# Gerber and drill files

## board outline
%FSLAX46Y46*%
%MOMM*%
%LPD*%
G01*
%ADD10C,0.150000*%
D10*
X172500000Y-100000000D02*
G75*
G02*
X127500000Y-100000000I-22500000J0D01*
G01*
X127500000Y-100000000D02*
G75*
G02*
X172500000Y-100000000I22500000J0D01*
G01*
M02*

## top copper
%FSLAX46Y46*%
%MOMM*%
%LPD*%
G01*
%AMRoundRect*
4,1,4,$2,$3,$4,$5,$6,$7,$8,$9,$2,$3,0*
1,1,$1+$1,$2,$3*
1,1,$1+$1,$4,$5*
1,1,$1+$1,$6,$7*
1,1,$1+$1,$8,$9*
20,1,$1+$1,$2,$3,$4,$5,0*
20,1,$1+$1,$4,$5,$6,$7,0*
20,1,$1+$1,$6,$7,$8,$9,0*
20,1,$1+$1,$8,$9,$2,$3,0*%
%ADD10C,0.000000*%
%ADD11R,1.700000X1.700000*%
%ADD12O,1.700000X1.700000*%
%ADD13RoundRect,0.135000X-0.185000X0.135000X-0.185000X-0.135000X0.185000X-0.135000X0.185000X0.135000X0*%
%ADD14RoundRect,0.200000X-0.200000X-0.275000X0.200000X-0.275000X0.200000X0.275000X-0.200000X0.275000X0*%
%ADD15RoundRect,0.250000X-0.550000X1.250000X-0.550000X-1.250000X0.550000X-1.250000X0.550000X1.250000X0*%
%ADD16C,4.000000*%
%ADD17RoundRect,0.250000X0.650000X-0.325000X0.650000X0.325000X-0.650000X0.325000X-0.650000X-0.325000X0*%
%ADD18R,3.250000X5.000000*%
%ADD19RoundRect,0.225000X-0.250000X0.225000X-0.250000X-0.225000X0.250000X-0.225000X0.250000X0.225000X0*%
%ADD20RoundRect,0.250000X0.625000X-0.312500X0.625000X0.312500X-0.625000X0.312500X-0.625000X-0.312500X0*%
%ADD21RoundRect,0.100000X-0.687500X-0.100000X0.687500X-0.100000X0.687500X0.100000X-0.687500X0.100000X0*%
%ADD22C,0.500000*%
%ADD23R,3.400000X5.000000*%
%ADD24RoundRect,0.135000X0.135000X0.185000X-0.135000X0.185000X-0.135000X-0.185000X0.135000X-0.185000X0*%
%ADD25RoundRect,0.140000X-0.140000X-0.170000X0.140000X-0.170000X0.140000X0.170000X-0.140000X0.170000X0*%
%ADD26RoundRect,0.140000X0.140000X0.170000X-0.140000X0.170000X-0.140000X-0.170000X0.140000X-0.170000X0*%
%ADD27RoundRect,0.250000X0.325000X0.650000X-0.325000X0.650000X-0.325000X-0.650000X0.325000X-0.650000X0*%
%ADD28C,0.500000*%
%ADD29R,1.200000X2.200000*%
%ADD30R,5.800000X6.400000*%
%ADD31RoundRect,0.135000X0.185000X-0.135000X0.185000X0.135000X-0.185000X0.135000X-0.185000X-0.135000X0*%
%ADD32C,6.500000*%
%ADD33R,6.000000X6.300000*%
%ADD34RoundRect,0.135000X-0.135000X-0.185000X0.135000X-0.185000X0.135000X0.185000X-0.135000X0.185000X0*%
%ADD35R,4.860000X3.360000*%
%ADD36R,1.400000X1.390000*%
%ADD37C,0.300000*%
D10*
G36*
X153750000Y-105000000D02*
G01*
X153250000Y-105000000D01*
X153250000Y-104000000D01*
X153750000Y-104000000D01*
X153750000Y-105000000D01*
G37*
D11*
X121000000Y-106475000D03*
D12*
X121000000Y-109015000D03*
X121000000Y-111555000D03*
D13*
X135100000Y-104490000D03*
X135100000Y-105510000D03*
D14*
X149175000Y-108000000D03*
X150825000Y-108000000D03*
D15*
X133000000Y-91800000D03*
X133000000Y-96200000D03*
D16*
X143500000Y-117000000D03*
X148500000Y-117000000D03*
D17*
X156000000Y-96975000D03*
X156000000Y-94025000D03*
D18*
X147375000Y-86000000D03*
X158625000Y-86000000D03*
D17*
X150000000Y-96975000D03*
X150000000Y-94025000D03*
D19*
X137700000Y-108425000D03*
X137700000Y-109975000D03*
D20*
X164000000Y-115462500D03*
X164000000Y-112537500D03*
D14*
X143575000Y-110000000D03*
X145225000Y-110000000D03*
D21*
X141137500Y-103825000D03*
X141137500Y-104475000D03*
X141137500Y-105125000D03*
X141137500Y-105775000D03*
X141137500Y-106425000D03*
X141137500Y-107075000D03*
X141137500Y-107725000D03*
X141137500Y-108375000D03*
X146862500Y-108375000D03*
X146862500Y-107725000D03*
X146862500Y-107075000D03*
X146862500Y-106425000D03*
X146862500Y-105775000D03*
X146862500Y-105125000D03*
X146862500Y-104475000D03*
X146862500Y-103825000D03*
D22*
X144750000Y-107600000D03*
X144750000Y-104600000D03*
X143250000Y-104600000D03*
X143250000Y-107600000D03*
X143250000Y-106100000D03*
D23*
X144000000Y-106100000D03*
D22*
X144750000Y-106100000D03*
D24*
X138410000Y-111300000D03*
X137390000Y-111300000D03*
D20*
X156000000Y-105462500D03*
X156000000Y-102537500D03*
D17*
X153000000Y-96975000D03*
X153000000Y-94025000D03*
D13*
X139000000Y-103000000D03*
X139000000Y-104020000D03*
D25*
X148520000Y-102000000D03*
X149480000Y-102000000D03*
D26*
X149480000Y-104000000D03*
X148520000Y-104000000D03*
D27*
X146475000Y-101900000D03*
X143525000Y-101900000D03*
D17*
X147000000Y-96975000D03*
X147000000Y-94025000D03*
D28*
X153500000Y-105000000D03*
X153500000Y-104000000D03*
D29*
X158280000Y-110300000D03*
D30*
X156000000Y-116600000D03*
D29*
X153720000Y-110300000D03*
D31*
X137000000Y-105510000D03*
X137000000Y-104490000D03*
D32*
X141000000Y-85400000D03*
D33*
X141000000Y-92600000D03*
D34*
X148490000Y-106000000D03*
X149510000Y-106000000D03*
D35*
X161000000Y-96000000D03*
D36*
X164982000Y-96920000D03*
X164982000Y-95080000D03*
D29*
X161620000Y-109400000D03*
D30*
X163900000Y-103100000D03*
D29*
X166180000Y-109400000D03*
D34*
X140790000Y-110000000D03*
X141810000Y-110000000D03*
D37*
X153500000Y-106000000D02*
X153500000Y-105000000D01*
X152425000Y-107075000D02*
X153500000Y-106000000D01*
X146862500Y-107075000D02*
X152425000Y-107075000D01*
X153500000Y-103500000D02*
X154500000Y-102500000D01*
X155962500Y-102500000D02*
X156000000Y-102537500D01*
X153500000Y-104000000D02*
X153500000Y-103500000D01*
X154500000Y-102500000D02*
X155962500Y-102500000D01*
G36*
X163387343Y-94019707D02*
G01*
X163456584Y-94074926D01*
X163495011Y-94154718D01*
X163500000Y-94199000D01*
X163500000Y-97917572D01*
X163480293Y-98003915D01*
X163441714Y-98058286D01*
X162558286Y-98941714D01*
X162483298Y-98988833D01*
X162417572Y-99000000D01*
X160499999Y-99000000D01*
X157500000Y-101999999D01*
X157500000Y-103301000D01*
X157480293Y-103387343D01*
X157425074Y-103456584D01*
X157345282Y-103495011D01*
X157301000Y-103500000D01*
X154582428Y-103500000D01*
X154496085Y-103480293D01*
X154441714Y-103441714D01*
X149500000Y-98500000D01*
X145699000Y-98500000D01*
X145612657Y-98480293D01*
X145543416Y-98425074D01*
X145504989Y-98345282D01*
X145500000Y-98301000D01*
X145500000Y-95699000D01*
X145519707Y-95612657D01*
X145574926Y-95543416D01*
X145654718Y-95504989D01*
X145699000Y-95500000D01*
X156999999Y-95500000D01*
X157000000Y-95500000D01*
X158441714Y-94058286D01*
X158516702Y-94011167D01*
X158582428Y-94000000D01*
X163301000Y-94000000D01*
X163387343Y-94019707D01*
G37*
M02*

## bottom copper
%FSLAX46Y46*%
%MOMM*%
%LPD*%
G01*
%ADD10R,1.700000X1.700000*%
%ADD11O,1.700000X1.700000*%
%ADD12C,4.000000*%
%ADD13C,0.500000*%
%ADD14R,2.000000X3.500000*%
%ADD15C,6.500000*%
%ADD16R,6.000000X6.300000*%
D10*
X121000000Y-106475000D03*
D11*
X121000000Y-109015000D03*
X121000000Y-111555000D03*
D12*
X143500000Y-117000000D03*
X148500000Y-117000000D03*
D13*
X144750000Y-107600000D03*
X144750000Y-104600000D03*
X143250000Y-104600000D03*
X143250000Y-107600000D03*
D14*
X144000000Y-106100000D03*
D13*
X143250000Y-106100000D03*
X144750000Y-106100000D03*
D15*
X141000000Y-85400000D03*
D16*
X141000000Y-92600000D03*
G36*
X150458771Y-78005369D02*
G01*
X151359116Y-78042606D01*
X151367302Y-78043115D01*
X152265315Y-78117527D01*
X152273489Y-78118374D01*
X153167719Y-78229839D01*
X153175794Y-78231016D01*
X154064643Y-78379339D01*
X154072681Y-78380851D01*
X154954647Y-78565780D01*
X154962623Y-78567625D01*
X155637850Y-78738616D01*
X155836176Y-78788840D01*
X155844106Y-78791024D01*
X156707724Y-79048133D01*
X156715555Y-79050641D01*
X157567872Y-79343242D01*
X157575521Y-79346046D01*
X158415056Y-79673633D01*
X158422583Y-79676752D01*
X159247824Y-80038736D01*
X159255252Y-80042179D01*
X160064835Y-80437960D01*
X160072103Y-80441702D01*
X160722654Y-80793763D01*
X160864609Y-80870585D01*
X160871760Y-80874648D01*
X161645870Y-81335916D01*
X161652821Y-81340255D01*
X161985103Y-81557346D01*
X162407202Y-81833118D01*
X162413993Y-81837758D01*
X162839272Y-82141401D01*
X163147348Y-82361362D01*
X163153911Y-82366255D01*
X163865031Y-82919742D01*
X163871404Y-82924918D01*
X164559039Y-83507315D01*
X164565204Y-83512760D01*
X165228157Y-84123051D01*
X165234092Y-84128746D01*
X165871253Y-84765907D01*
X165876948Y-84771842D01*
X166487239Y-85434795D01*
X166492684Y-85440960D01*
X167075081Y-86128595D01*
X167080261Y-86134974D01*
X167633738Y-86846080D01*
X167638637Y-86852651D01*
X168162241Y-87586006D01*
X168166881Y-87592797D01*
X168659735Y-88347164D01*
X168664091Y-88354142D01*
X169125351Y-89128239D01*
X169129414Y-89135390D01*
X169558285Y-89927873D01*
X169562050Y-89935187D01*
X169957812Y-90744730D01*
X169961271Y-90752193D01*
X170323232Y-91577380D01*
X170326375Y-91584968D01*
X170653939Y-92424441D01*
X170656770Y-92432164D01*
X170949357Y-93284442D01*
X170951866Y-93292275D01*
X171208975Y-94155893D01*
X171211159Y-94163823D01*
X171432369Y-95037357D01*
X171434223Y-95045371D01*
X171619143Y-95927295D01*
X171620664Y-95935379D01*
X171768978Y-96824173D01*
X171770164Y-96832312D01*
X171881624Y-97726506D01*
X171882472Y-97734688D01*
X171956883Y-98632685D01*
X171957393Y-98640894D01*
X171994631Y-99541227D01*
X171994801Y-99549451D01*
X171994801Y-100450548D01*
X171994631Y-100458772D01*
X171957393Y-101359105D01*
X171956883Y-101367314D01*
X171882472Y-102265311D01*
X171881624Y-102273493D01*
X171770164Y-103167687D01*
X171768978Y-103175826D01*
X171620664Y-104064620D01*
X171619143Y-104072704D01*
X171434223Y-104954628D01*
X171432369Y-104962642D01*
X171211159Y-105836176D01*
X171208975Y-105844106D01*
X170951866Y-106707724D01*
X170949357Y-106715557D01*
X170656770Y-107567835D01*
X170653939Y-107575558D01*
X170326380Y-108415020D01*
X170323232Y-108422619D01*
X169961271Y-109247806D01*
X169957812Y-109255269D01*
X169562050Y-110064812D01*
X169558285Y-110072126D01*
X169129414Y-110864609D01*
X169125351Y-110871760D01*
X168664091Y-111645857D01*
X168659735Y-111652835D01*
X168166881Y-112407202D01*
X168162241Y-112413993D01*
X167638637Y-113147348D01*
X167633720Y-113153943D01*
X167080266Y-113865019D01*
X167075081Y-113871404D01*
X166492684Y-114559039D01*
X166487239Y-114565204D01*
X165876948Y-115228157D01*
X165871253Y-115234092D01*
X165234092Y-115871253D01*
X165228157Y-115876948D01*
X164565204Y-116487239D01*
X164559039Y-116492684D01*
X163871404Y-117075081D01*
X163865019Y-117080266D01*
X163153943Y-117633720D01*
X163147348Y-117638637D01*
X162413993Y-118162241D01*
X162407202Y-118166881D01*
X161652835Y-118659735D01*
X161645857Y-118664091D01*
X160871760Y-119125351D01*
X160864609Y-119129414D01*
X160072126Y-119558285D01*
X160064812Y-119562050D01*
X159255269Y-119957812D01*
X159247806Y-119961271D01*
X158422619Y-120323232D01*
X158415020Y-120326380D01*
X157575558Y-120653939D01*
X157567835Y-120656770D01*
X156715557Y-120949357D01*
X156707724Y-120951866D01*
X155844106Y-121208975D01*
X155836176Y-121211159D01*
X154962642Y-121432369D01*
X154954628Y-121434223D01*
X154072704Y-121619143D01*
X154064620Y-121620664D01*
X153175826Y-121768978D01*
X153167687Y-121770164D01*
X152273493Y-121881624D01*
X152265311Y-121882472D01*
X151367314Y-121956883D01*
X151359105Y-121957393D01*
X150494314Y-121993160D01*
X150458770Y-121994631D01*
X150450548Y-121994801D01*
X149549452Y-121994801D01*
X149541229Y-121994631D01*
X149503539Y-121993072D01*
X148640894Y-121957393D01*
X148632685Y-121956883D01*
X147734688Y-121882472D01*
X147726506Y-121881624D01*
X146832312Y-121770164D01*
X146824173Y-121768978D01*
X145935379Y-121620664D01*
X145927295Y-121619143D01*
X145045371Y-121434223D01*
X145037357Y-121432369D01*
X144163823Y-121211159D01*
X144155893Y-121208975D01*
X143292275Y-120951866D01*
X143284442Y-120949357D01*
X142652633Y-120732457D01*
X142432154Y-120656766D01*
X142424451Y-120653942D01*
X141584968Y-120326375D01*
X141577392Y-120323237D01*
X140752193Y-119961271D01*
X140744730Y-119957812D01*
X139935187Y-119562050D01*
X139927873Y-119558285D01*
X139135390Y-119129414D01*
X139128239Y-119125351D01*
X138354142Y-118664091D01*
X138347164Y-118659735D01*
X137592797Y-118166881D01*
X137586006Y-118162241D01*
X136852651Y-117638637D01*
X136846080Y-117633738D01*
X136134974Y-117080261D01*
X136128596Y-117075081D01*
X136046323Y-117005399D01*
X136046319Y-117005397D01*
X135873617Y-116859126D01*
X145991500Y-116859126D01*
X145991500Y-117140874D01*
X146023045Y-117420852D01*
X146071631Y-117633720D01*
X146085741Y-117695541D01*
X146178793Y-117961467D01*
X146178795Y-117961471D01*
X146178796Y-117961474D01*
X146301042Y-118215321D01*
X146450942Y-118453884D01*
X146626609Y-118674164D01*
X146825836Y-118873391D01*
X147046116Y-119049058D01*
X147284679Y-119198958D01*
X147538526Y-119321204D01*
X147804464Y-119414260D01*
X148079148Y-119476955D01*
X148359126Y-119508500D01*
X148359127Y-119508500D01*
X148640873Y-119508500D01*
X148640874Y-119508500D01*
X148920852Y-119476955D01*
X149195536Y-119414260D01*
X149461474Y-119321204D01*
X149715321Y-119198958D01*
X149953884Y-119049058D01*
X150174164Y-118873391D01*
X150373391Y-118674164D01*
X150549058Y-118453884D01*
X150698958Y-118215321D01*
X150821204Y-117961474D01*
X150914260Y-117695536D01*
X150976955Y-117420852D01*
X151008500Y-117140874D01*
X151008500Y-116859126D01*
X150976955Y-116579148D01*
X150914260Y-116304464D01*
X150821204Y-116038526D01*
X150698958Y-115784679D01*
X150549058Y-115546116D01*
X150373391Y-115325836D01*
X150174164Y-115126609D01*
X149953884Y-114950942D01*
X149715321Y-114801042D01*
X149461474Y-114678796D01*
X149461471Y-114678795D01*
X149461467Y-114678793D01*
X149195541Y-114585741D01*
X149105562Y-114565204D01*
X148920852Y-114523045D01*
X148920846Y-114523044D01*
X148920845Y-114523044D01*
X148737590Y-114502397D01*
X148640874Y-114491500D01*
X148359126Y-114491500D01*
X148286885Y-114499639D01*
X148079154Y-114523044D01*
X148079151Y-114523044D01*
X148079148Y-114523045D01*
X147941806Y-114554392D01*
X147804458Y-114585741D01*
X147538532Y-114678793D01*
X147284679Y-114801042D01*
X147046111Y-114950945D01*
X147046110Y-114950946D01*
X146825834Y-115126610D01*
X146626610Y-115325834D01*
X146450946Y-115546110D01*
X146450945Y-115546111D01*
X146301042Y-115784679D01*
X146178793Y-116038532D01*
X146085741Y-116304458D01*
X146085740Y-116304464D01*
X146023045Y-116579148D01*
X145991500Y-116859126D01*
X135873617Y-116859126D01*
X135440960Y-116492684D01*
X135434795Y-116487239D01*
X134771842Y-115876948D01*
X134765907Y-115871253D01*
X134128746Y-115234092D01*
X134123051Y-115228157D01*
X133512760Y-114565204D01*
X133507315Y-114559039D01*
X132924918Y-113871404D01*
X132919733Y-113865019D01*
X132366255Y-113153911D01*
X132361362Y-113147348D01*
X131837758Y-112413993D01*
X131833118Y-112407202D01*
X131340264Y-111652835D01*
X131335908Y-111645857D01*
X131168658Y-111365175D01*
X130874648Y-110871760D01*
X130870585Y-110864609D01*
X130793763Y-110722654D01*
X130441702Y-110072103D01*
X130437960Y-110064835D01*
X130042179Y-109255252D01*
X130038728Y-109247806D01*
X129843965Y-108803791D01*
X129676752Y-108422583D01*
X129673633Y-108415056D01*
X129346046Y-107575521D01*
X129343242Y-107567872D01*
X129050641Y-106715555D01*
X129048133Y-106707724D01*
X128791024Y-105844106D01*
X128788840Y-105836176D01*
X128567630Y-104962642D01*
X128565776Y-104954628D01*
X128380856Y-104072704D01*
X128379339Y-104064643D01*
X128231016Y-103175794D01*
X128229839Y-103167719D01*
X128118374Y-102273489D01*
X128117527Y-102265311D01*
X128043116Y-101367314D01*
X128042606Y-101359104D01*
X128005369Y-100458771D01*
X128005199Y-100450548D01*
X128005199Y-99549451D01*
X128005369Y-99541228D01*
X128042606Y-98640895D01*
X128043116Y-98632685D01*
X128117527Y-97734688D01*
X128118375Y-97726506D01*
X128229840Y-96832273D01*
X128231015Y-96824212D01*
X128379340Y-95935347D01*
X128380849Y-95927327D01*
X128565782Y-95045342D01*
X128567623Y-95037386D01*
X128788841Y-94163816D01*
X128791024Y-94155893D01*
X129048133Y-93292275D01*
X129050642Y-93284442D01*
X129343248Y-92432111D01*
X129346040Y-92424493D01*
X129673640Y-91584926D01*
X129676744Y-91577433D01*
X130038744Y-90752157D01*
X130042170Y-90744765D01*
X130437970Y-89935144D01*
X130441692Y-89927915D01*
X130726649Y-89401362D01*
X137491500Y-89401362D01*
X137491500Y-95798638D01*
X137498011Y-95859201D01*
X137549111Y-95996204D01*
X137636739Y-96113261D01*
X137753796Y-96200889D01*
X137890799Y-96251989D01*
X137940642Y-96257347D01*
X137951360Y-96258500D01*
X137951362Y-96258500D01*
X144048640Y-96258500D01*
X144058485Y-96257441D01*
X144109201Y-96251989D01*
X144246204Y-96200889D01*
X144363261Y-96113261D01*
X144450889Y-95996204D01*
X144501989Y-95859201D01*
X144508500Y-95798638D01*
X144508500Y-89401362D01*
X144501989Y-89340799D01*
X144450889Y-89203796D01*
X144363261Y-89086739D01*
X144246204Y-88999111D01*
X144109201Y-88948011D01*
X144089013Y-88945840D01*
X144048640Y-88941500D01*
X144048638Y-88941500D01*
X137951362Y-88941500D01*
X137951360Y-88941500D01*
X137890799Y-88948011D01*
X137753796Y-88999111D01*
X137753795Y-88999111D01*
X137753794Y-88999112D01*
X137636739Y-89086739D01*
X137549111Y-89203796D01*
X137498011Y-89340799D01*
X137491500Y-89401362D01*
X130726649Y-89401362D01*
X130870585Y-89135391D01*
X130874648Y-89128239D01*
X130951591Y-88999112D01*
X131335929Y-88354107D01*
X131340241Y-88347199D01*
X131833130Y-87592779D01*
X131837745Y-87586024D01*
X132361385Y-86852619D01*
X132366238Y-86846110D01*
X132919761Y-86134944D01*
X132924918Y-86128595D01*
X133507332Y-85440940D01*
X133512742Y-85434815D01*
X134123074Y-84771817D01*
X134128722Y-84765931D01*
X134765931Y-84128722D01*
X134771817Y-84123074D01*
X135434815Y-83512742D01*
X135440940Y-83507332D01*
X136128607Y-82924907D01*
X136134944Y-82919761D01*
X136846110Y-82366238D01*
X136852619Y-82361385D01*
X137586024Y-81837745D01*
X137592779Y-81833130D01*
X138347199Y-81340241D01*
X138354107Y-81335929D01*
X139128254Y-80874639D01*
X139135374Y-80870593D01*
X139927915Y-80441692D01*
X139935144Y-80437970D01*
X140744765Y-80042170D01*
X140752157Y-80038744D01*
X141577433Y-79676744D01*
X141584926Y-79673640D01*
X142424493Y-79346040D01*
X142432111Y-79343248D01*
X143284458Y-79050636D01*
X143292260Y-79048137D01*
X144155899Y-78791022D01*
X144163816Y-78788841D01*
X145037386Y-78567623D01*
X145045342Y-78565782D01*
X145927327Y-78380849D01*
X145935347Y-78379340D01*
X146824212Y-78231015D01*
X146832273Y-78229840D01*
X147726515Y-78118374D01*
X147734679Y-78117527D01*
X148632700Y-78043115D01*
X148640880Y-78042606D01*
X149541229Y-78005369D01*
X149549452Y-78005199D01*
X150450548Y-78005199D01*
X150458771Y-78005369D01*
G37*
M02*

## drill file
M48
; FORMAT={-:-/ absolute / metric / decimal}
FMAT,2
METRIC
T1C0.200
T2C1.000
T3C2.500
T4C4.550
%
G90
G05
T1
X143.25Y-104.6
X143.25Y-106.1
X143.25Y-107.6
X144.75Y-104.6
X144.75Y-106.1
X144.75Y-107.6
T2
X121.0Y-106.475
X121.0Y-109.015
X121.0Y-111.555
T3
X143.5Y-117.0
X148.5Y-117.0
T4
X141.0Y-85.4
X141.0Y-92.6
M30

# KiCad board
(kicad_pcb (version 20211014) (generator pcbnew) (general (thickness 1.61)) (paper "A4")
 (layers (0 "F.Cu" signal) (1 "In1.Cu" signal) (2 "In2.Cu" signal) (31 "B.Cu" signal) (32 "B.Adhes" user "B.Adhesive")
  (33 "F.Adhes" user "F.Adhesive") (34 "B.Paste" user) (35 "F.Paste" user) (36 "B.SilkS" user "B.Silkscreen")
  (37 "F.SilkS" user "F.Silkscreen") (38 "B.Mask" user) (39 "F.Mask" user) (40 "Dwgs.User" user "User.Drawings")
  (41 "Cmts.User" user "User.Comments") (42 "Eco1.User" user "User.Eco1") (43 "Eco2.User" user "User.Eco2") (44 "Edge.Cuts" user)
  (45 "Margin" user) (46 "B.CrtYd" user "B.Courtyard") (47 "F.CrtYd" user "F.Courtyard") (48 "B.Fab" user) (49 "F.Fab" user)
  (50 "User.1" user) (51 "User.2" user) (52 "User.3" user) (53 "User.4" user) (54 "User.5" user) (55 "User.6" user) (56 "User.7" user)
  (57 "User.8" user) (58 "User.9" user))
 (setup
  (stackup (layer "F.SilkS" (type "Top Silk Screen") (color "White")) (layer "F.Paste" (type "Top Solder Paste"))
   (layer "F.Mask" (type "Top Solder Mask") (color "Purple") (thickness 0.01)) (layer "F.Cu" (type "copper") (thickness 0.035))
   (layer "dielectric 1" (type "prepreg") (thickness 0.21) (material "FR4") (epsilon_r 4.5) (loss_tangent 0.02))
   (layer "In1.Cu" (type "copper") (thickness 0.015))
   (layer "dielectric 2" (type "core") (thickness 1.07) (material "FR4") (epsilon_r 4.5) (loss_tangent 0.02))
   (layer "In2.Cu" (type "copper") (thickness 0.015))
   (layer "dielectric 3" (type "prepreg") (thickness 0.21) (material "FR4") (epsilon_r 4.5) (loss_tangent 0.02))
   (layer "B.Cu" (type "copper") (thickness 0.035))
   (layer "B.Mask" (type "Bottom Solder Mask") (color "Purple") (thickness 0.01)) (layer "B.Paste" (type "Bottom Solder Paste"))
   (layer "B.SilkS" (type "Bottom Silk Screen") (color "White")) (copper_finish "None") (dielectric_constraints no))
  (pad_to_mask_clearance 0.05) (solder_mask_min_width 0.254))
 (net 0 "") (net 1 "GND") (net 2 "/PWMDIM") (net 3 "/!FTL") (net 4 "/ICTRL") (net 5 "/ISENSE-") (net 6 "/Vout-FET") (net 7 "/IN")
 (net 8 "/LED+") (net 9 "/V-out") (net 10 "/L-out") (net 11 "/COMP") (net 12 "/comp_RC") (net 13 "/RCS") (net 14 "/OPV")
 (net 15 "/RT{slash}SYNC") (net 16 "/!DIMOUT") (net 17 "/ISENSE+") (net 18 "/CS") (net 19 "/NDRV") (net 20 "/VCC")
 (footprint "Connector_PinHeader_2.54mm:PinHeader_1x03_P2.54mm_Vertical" (layer "F.Cu") (at 121 106.475)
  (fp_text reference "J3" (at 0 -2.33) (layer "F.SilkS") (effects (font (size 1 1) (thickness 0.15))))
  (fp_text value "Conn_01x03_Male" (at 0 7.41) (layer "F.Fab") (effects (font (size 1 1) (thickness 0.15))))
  (pad "1" thru_hole rect (at 0 0) (size 1.7 1.7) (drill 1) (layers *.Cu *.Mask) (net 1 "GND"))
  (pad "2" thru_hole oval (at 0 2.54) (size 1.7 1.7) (drill 1) (layers *.Cu *.Mask) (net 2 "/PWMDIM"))
  (pad "3" thru_hole oval (at 0 5.08) (size 1.7 1.7) (drill 1) (layers *.Cu *.Mask) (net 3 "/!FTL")))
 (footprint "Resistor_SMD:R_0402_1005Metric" (layer "F.Cu") (at 135.1 105 -90)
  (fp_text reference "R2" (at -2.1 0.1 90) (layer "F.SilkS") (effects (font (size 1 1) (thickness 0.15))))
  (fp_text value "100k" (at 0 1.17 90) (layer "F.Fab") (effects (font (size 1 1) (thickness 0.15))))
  (pad "1" smd roundrect (at -0.51 0 270) (size 0.54 0.64) (layers "F.Cu" "F.Paste" "F.Mask") (roundrect_rratio 0.25) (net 1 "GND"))
  (pad "2" smd roundrect (at 0.51 0 270) (size 0.54 0.64) (layers "F.Cu" "F.Paste" "F.Mask") (roundrect_rratio 0.25) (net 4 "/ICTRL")))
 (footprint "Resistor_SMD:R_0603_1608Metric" (layer "F.Cu") (at 150 108)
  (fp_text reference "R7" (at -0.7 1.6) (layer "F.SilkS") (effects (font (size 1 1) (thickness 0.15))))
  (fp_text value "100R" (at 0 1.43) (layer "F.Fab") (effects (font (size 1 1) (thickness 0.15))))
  (pad "1" smd roundrect (at -0.825 0) (size 0.8 0.95) (layers "F.Cu" "F.Paste" "F.Mask") (roundrect_rratio 0.25) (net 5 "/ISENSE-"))
  (pad "2" smd roundrect (at 0.825 0) (size 0.8 0.95) (layers "F.Cu" "F.Paste" "F.Mask") (roundrect_rratio 0.25) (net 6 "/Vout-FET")))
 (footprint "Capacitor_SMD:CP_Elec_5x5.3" (layer "F.Cu") (at 133 94 -90)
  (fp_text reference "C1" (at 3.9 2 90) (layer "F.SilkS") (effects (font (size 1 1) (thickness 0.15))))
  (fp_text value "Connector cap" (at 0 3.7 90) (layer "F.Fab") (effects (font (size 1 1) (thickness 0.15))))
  (pad "1" smd roundrect (at -2.2 0 270) (size 3 1.6) (layers "F.Cu" "F.Paste" "F.Mask") (roundrect_rratio 0.15625) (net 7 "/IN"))
  (pad "2" smd roundrect (at 2.2 0 270) (size 3 1.6) (layers "F.Cu" "F.Paste" "F.Mask") (roundrect_rratio 0.15625) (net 1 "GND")))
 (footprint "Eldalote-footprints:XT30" (layer "F.Cu") (at 146 117)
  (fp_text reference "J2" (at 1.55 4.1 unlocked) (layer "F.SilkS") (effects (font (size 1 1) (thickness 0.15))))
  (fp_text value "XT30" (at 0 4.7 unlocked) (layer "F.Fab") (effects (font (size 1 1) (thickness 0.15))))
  (pad "1" thru_hole circle (at -2.5 0) (size 4 4) (drill 2.5) (layers *.Cu *.Mask) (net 1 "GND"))
  (pad "2" thru_hole circle (at 2.5 0) (size 4 4) (drill 2.5) (layers *.Cu *.Mask) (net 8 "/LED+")))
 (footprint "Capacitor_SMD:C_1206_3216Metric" (layer "F.Cu") (at 156 95.5 90)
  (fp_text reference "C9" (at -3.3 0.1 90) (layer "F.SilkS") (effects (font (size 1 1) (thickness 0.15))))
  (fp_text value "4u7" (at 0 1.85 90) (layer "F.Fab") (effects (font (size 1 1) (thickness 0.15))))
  (pad "1" smd roundrect (at -1.475 0 90) (size 1.15 1.8) (layers "F.Cu" "F.Paste" "F.Mask") (roundrect_rratio 0.217391) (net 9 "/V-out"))
  (pad "2" smd roundrect (at 1.475 0 90) (size 1.15 1.8) (layers "F.Cu" "F.Paste" "F.Mask") (roundrect_rratio 0.217391) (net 1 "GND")))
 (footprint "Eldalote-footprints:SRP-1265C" (layer "F.Cu") (at 153 86)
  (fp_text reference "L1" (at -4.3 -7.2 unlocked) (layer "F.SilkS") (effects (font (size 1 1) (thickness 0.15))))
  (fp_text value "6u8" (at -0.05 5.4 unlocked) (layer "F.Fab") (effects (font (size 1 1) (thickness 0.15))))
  (pad "1" smd rect (at -5.625 0) (size 3.25 5) (layers "F.Cu" "F.Paste" "F.Mask") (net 7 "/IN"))
  (pad "2" smd rect (at 5.625 0) (size 3.25 5) (layers "F.Cu" "F.Paste" "F.Mask") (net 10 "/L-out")))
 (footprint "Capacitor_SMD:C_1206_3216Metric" (layer "F.Cu") (at 150 95.5 90)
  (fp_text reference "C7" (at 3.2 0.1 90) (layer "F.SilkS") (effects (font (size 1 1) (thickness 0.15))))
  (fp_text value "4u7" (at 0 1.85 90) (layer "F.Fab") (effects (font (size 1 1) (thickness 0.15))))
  (pad "1" smd roundrect (at -1.475 0 90) (size 1.15 1.8) (layers "F.Cu" "F.Paste" "F.Mask") (roundrect_rratio 0.217391) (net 9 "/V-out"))
  (pad "2" smd roundrect (at 1.475 0 90) (size 1.15 1.8) (layers "F.Cu" "F.Paste" "F.Mask") (roundrect_rratio 0.217391) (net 1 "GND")))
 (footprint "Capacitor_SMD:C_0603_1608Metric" (layer "F.Cu") (at 137.7 109.2 -90)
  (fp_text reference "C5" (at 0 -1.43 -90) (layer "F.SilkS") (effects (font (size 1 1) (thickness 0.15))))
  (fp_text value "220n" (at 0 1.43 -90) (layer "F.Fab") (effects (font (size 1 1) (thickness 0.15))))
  (pad "1" smd roundrect (at -0.775 0 270) (size 0.9 0.95) (layers "F.Cu" "F.Paste" "F.Mask") (roundrect_rratio 0.25) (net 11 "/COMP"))
  (pad "2" smd roundrect (at 0.775 0 270) (size 0.9 0.95) (layers "F.Cu" "F.Paste" "F.Mask") (roundrect_rratio 0.25) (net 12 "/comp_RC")))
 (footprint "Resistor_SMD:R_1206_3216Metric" (layer "F.Cu") (at 164 114 90)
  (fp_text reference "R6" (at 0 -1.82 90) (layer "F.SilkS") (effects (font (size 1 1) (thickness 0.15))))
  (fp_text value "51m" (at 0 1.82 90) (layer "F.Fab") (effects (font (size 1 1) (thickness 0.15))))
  (pad "1" smd roundrect (at -1.4625 0 90) (size 1.125 1.75) (layers "F.Cu" "F.Paste" "F.Mask") (roundrect_rratio 0.222222) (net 1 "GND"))
  (pad "2" smd roundrect (at 1.4625 0 90) (size 1.125 1.75) (layers "F.Cu" "F.Paste" "F.Mask") (roundrect_rratio 0.222222) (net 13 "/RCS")))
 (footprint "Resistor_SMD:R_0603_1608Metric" (layer "F.Cu") (at 144.4 110)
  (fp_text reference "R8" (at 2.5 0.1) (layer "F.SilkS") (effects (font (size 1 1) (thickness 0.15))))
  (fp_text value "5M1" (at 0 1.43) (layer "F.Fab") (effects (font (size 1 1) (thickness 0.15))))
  (pad "1" smd roundrect (at -0.825 0) (size 0.8 0.95) (layers "F.Cu" "F.Paste" "F.Mask") (roundrect_rratio 0.25) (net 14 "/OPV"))
  (pad "2" smd roundrect (at 0.825 0) (size 0.8 0.95) (layers "F.Cu" "F.Paste" "F.Mask") (roundrect_rratio 0.25) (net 9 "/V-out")))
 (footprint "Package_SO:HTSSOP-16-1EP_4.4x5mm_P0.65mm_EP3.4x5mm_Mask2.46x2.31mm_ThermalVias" (layer "F.Cu") (at 144 106.1)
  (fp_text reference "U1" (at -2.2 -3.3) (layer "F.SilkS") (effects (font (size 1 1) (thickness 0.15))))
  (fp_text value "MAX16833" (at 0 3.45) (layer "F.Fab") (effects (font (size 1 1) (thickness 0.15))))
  (pad "" smd rect (at 0 0) (size 2.46 2.31) (layers "F.Mask"))
  (pad "" smd roundrect (at 0 0.58) (size 1.98 0.93) (layers "F.Paste") (roundrect_rratio 0.25))
  (pad "" smd roundrect (at 0 -0.58) (size 1.98 0.93) (layers "F.Paste") (roundrect_rratio 0.25))
  (pad "1" smd roundrect (at -2.8625 -2.275) (size 1.575 0.4) (layers "F.Cu" "F.Paste" "F.Mask") (roundrect_rratio 0.25) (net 1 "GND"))
  (pad "2" smd roundrect (at -2.8625 -1.625) (size 1.575 0.4) (layers "F.Cu" "F.Paste" "F.Mask") (roundrect_rratio 0.25)
   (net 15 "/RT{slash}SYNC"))
  (pad "3" smd roundrect (at -2.8625 -0.975) (size 1.575 0.4) (layers "F.Cu" "F.Paste" "F.Mask") (roundrect_rratio 0.25) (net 1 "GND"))
  (pad "4" smd roundrect (at -2.8625 -0.325) (size 1.575 0.4) (layers "F.Cu" "F.Paste" "F.Mask") (roundrect_rratio 0.25) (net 4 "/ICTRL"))
  (pad "5" smd roundrect (at -2.8625 0.325) (size 1.575 0.4) (layers "F.Cu" "F.Paste" "F.Mask") (roundrect_rratio 0.25) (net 11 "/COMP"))
  (pad "6" smd roundrect (at -2.8625 0.975) (size 1.575 0.4) (layers "F.Cu" "F.Paste" "F.Mask") (roundrect_rratio 0.25) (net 3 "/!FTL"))
  (pad "7" smd roundrect (at -2.8625 1.625) (size 1.575 0.4) (layers "F.Cu" "F.Paste" "F.Mask") (roundrect_rratio 0.25) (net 2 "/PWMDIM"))
  (pad "8" smd roundrect (at -2.8625 2.275) (size 1.575 0.4) (layers "F.Cu" "F.Paste" "F.Mask") (roundrect_rratio 0.25) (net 14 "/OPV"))
  (pad "9" smd roundrect (at 2.8625 2.275) (size 1.575 0.4) (layers "F.Cu" "F.Paste" "F.Mask") (roundrect_rratio 0.25) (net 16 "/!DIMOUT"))
  (pad "10" smd roundrect (at 2.8625 1.625) (size 1.575 0.4) (layers "F.Cu" "F.Paste" "F.Mask") (roundrect_rratio 0.25) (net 5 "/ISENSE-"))
  (pad "11" smd roundrect (at 2.8625 0.975) (size 1.575 0.4) (layers "F.Cu" "F.Paste" "F.Mask") (roundrect_rratio 0.25) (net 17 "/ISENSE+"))
  (pad "12" smd roundrect (at 2.8625 0.325) (size 1.575 0.4) (layers "F.Cu" "F.Paste" "F.Mask") (roundrect_rratio 0.25) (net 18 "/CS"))
  (pad "13" smd roundrect (at 2.8625 -0.325) (size 1.575 0.4) (layers "F.Cu" "F.Paste" "F.Mask") (roundrect_rratio 0.25) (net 1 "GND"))
  (pad "14" smd roundrect (at 2.8625 -0.975) (size 1.575 0.4) (layers "F.Cu" "F.Paste" "F.Mask") (roundrect_rratio 0.25) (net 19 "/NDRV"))
  (pad "15" smd roundrect (at 2.8625 -1.625) (size 1.575 0.4) (layers "F.Cu" "F.Paste" "F.Mask") (roundrect_rratio 0.25) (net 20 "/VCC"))
  (pad "16" smd roundrect (at 2.8625 -2.275) (size 1.575 0.4) (layers "F.Cu" "F.Paste" "F.Mask") (roundrect_rratio 0.25) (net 7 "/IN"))
  (pad "17" thru_hole circle (at 0.75 1.5) (size 0.5 0.5) (drill 0.2) (layers *.Cu) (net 1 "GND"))
  (pad "17" thru_hole circle (at 0.75 -1.5) (size 0.5 0.5) (drill 0.2) (layers *.Cu) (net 1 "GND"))
  (pad "17" thru_hole circle (at -0.75 -1.5) (size 0.5 0.5) (drill 0.2) (layers *.Cu) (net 1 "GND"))
  (pad "17" thru_hole circle (at -0.75 1.5) (size 0.5 0.5) (drill 0.2) (layers *.Cu) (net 1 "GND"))
  (pad "17" smd rect (at 0 0) (size 2 3.5) (layers "B.Cu") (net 1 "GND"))
  (pad "17" thru_hole circle (at -0.75 0) (size 0.5 0.5) (drill 0.2) (layers *.Cu) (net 1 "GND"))
  (pad "17" smd rect (at 0 0) (size 3.4 5) (layers "F.Cu") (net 1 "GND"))
  (pad "17" thru_hole circle (at 0.75 0) (size 0.5 0.5) (drill 0.2) (layers *.Cu) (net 1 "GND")))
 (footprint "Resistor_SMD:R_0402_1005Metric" (layer "F.Cu") (at 137.9 111.3 180)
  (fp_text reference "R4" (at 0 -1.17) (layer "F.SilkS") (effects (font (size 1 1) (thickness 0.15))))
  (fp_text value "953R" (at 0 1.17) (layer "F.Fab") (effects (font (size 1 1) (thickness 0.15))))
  (pad "1" smd roundrect (at -0.51 0 180) (size 0.54 0.64) (layers "F.Cu" "F.Paste" "F.Mask") (roundrect_rratio 0.25) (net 1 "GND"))
  (pad "2" smd roundrect (at 0.51 0 180) (size 0.54 0.64) (layers "F.Cu" "F.Paste" "F.Mask") (roundrect_rratio 0.25) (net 12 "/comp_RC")))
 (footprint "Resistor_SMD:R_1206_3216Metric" (layer "F.Cu") (at 156 104 90)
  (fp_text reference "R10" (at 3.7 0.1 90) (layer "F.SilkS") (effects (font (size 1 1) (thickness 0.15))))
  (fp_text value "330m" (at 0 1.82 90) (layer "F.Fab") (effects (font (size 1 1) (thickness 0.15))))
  (pad "1" smd roundrect (at -1.4625 0 90) (size 1.125 1.75) (layers "F.Cu" "F.Paste" "F.Mask") (roundrect_rratio 0.222222)
   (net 6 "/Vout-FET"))
  (pad "2" smd roundrect (at 1.4625 0 90) (size 1.125 1.75) (layers "F.Cu" "F.Paste" "F.Mask") (roundrect_rratio 0.222222) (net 9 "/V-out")))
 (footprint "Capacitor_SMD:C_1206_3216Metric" (layer "F.Cu") (at 153 95.5 90)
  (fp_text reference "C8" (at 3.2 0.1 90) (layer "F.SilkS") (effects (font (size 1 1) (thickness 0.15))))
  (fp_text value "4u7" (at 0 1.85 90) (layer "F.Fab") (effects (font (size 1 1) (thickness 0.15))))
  (pad "1" smd roundrect (at -1.475 0 90) (size 1.15 1.8) (layers "F.Cu" "F.Paste" "F.Mask") (roundrect_rratio 0.217391) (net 9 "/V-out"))
  (pad "2" smd roundrect (at 1.475 0 90) (size 1.15 1.8) (layers "F.Cu" "F.Paste" "F.Mask") (roundrect_rratio 0.217391) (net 1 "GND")))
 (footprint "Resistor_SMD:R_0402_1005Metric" (layer "F.Cu") (at 139 103.51 -90)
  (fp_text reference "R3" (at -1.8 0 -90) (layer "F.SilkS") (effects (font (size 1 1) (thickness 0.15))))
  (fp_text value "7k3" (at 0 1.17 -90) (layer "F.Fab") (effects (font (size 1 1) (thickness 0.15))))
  (pad "1" smd roundrect (at -0.51 0 270) (size 0.54 0.64) (layers "F.Cu" "F.Paste" "F.Mask") (roundrect_rratio 0.25) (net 1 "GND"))
  (pad "2" smd roundrect (at 0.51 0 270) (size 0.54 0.64) (layers "F.Cu" "F.Paste" "F.Mask") (roundrect_rratio 0.25)
   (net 15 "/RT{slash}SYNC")))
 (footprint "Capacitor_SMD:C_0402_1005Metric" (layer "F.Cu") (at 149 102)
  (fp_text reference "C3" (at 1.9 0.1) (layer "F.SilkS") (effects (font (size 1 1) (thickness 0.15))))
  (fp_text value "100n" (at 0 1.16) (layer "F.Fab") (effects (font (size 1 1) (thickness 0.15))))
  (pad "1" smd roundrect (at -0.48 0) (size 0.56 0.62) (layers "F.Cu" "F.Paste" "F.Mask") (roundrect_rratio 0.25) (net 7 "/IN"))
  (pad "2" smd roundrect (at 0.48 0) (size 0.56 0.62) (layers "F.Cu" "F.Paste" "F.Mask") (roundrect_rratio 0.25) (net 1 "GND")))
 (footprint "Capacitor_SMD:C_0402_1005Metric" (layer "F.Cu") (at 149 104 180)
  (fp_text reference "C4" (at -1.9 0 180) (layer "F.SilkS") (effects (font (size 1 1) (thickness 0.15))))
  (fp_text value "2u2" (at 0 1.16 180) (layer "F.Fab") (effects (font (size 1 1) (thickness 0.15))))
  (pad "1" smd roundrect (at -0.48 0 180) (size 0.56 0.62) (layers "F.Cu" "F.Paste" "F.Mask") (roundrect_rratio 0.25) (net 1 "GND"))
  (pad "2" smd roundrect (at 0.48 0 180) (size 0.56 0.62) (layers "F.Cu" "F.Paste" "F.Mask") (roundrect_rratio 0.25) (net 20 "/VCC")))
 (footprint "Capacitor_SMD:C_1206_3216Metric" (layer "F.Cu") (at 145 101.9 180)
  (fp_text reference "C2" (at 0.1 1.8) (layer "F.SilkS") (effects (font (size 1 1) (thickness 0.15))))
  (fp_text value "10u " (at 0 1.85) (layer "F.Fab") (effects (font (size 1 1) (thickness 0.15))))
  (pad "1" smd roundrect (at -1.475 0 180) (size 1.15 1.8) (layers "F.Cu" "F.Paste" "F.Mask") (roundrect_rratio 0.217391) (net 7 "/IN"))
  (pad "2" smd roundrect (at 1.475 0 180) (size 1.15 1.8) (layers "F.Cu" "F.Paste" "F.Mask") (roundrect_rratio 0.217391) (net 1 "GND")))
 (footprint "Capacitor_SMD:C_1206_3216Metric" (layer "F.Cu") (at 147 95.5 90)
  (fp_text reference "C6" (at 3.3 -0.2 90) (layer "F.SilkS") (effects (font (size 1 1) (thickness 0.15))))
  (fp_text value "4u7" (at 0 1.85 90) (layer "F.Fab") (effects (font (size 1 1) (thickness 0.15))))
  (pad "1" smd roundrect (at -1.475 0 90) (size 1.15 1.8) (layers "F.Cu" "F.Paste" "F.Mask") (roundrect_rratio 0.217391) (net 9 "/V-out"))
  (pad "2" smd roundrect (at 1.475 0 90) (size 1.15 1.8) (layers "F.Cu" "F.Paste" "F.Mask") (roundrect_rratio 0.217391) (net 1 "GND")))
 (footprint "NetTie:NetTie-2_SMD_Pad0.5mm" (layer "F.Cu") (at 153.5 104.5 90)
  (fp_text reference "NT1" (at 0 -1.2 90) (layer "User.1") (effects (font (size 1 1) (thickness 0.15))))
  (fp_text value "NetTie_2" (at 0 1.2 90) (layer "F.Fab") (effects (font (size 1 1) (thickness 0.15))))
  (fp_poly (pts (xy -0.5 -0.25) (xy 0.5 -0.25) (xy 0.5 0.25) (xy -0.5 0.25)) (layer "F.Cu") (width 0) (fill solid))
  (pad "1" smd circle (at -0.5 0 90) (size 0.5 0.5) (layers "F.Cu") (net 17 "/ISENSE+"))
  (pad "2" smd circle (at 0.5 0 90) (size 0.5 0.5) (layers "F.Cu") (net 9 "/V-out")))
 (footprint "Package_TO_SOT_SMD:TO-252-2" (layer "F.Cu") (at 156 114.5 -90)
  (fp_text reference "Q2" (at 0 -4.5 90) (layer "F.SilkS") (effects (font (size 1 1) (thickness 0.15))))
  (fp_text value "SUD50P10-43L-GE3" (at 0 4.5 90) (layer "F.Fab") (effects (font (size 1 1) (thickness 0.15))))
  (pad "" smd rect (at 0.425 -1.525 270) (size 3.05 2.75) (layers "F.Paste"))
  (pad "" smd rect (at 3.775 1.525 270) (size 3.05 2.75) (layers "F.Paste"))
  (pad "" smd rect (at 0.425 1.525 270) (size 3.05 2.75) (layers "F.Paste"))
  (pad "" smd rect (at 3.775 -1.525 270) (size 3.05 2.75) (layers "F.Paste"))
  (pad "1" smd rect (at -4.2 -2.28 270) (size 2.2 1.2) (layers "F.Cu" "F.Paste" "F.Mask") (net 16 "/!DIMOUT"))
  (pad "2" smd rect (at 2.1 0 270) (size 6.4 5.8) (layers "F.Cu" "F.Mask") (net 8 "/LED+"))
  (pad "3" smd rect (at -4.2 2.28 270) (size 2.2 1.2) (layers "F.Cu" "F.Paste" "F.Mask") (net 6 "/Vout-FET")))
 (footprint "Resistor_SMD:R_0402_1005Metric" (layer "F.Cu") (at 137 105 90)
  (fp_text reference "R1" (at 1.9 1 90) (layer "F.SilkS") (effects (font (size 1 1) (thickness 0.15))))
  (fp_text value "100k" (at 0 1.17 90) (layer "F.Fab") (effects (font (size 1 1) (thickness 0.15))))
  (pad "1" smd roundrect (at -0.51 0 90) (size 0.54 0.64) (layers "F.Cu" "F.Paste" "F.Mask") (roundrect_rratio 0.25) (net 4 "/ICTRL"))
  (pad "2" smd roundrect (at 0.51 0 90) (size 0.54 0.64) (layers "F.Cu" "F.Paste" "F.Mask") (roundrect_rratio 0.25) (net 20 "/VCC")))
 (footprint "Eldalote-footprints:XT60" (layer "F.Cu") (at 141 89 -90)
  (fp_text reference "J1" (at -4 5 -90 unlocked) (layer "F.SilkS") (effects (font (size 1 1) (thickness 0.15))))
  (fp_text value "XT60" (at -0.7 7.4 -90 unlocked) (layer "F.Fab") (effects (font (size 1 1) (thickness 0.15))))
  (pad "N" thru_hole circle (at -3.6 0 270) (size 6.5 6.5) (drill 4.55) (layers *.Cu *.Mask) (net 1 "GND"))
  (pad "P" thru_hole rect (at 3.6 0 270) (size 6.3 6) (drill 4.55) (layers *.Cu *.Mask) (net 7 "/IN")))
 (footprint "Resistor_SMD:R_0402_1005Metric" (layer "F.Cu") (at 149 106)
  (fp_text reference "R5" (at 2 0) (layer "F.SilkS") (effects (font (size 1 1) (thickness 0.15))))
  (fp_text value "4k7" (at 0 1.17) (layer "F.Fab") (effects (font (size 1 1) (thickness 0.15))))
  (pad "1" smd roundrect (at -0.51 0) (size 0.54 0.64) (layers "F.Cu" "F.Paste" "F.Mask") (roundrect_rratio 0.25) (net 18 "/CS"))
  (pad "2" smd roundrect (at 0.51 0) (size 0.54 0.64) (layers "F.Cu" "F.Paste" "F.Mask") (roundrect_rratio 0.25) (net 13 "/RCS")))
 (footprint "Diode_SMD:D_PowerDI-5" (layer "F.Cu") (at 162.12 96)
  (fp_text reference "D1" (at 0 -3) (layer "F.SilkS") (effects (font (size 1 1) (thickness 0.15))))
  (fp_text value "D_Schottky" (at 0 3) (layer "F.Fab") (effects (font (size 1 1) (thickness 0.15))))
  (pad "1" smd rect (at -1.12 0 180) (size 4.86 3.36) (layers "F.Cu" "F.Paste" "F.Mask") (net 9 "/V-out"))
  (pad "2" smd rect (at 2.862 0.92 180) (size 1.4 1.39) (layers "F.Cu" "F.Paste" "F.Mask") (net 10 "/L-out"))
  (pad "2" smd rect (at 2.862 -0.92 180) (size 1.4 1.39) (layers "F.Cu" "F.Paste" "F.Mask") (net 10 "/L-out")))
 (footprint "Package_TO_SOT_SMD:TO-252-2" (layer "F.Cu") (at 163.9 105.2 90)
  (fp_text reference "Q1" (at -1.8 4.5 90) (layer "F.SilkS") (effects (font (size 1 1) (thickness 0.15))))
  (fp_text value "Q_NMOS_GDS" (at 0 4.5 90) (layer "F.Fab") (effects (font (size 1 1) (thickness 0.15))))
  (pad "" smd rect (at 0.425 -1.525 90) (size 3.05 2.75) (layers "F.Paste"))
  (pad "" smd rect (at 0.425 1.525 90) (size 3.05 2.75) (layers "F.Paste"))
  (pad "" smd rect (at 3.775 1.525 90) (size 3.05 2.75) (layers "F.Paste"))
  (pad "" smd rect (at 3.775 -1.525 90) (size 3.05 2.75) (layers "F.Paste"))
  (pad "1" smd rect (at -4.2 -2.28 90) (size 2.2 1.2) (layers "F.Cu" "F.Paste" "F.Mask") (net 19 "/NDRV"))
  (pad "2" smd rect (at 2.1 0 90) (size 6.4 5.8) (layers "F.Cu" "F.Mask") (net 10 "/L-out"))
  (pad "3" smd rect (at -4.2 2.28 90) (size 2.2 1.2) (layers "F.Cu" "F.Paste" "F.Mask") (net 13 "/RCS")))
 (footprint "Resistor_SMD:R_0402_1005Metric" (layer "F.Cu") (at 141.3 110)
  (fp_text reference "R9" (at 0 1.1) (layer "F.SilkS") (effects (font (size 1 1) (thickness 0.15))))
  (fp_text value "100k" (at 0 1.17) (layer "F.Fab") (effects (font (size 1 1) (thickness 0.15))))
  (pad "1" smd roundrect (at -0.51 0) (size 0.54 0.64) (layers "F.Cu" "F.Paste" "F.Mask") (roundrect_rratio 0.25) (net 1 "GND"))
  (pad "2" smd roundrect (at 0.51 0) (size 0.54 0.64) (layers "F.Cu" "F.Paste" "F.Mask") (roundrect_rratio 0.25) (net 14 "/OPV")))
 (gr_circle locked (center 150 100) (end 172.5 100) (layer "Edge.Cuts") (width 0.15) (fill none))
 (segment (start 153.5 106) (end 153.5 105) (width 0.3) (layer "F.Cu") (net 17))
 (segment (start 152.425 107.075) (end 153.5 106) (width 0.3) (layer "F.Cu") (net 17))
 (segment (start 146.8625 107.075) (end 152.425 107.075) (width 0.3) (layer "F.Cu") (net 17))
 (segment (start 153.5 103.5) (end 154.5 102.5) (width 0.3) (layer "F.Cu") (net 9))
 (segment (start 155.9625 102.5) (end 156 102.5375) (width 0.3) (layer "F.Cu") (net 9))
 (segment (start 153.5 104) (end 153.5 103.5) (width 0.3) (layer "F.Cu") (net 9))
 (segment (start 154.5 102.5) (end 155.9625 102.5) (width 0.3) (layer "F.Cu") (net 9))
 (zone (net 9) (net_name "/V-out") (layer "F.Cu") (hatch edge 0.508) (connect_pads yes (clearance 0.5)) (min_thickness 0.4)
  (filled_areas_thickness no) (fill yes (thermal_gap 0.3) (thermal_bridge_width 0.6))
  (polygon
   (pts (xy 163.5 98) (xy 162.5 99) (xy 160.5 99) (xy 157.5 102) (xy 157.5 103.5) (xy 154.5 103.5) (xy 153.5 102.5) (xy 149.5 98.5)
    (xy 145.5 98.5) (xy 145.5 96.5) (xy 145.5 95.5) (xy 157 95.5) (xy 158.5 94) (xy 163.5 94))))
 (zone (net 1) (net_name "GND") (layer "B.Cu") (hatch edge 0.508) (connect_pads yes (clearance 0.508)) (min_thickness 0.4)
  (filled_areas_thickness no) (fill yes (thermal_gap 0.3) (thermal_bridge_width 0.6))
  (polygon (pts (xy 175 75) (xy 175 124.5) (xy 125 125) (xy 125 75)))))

